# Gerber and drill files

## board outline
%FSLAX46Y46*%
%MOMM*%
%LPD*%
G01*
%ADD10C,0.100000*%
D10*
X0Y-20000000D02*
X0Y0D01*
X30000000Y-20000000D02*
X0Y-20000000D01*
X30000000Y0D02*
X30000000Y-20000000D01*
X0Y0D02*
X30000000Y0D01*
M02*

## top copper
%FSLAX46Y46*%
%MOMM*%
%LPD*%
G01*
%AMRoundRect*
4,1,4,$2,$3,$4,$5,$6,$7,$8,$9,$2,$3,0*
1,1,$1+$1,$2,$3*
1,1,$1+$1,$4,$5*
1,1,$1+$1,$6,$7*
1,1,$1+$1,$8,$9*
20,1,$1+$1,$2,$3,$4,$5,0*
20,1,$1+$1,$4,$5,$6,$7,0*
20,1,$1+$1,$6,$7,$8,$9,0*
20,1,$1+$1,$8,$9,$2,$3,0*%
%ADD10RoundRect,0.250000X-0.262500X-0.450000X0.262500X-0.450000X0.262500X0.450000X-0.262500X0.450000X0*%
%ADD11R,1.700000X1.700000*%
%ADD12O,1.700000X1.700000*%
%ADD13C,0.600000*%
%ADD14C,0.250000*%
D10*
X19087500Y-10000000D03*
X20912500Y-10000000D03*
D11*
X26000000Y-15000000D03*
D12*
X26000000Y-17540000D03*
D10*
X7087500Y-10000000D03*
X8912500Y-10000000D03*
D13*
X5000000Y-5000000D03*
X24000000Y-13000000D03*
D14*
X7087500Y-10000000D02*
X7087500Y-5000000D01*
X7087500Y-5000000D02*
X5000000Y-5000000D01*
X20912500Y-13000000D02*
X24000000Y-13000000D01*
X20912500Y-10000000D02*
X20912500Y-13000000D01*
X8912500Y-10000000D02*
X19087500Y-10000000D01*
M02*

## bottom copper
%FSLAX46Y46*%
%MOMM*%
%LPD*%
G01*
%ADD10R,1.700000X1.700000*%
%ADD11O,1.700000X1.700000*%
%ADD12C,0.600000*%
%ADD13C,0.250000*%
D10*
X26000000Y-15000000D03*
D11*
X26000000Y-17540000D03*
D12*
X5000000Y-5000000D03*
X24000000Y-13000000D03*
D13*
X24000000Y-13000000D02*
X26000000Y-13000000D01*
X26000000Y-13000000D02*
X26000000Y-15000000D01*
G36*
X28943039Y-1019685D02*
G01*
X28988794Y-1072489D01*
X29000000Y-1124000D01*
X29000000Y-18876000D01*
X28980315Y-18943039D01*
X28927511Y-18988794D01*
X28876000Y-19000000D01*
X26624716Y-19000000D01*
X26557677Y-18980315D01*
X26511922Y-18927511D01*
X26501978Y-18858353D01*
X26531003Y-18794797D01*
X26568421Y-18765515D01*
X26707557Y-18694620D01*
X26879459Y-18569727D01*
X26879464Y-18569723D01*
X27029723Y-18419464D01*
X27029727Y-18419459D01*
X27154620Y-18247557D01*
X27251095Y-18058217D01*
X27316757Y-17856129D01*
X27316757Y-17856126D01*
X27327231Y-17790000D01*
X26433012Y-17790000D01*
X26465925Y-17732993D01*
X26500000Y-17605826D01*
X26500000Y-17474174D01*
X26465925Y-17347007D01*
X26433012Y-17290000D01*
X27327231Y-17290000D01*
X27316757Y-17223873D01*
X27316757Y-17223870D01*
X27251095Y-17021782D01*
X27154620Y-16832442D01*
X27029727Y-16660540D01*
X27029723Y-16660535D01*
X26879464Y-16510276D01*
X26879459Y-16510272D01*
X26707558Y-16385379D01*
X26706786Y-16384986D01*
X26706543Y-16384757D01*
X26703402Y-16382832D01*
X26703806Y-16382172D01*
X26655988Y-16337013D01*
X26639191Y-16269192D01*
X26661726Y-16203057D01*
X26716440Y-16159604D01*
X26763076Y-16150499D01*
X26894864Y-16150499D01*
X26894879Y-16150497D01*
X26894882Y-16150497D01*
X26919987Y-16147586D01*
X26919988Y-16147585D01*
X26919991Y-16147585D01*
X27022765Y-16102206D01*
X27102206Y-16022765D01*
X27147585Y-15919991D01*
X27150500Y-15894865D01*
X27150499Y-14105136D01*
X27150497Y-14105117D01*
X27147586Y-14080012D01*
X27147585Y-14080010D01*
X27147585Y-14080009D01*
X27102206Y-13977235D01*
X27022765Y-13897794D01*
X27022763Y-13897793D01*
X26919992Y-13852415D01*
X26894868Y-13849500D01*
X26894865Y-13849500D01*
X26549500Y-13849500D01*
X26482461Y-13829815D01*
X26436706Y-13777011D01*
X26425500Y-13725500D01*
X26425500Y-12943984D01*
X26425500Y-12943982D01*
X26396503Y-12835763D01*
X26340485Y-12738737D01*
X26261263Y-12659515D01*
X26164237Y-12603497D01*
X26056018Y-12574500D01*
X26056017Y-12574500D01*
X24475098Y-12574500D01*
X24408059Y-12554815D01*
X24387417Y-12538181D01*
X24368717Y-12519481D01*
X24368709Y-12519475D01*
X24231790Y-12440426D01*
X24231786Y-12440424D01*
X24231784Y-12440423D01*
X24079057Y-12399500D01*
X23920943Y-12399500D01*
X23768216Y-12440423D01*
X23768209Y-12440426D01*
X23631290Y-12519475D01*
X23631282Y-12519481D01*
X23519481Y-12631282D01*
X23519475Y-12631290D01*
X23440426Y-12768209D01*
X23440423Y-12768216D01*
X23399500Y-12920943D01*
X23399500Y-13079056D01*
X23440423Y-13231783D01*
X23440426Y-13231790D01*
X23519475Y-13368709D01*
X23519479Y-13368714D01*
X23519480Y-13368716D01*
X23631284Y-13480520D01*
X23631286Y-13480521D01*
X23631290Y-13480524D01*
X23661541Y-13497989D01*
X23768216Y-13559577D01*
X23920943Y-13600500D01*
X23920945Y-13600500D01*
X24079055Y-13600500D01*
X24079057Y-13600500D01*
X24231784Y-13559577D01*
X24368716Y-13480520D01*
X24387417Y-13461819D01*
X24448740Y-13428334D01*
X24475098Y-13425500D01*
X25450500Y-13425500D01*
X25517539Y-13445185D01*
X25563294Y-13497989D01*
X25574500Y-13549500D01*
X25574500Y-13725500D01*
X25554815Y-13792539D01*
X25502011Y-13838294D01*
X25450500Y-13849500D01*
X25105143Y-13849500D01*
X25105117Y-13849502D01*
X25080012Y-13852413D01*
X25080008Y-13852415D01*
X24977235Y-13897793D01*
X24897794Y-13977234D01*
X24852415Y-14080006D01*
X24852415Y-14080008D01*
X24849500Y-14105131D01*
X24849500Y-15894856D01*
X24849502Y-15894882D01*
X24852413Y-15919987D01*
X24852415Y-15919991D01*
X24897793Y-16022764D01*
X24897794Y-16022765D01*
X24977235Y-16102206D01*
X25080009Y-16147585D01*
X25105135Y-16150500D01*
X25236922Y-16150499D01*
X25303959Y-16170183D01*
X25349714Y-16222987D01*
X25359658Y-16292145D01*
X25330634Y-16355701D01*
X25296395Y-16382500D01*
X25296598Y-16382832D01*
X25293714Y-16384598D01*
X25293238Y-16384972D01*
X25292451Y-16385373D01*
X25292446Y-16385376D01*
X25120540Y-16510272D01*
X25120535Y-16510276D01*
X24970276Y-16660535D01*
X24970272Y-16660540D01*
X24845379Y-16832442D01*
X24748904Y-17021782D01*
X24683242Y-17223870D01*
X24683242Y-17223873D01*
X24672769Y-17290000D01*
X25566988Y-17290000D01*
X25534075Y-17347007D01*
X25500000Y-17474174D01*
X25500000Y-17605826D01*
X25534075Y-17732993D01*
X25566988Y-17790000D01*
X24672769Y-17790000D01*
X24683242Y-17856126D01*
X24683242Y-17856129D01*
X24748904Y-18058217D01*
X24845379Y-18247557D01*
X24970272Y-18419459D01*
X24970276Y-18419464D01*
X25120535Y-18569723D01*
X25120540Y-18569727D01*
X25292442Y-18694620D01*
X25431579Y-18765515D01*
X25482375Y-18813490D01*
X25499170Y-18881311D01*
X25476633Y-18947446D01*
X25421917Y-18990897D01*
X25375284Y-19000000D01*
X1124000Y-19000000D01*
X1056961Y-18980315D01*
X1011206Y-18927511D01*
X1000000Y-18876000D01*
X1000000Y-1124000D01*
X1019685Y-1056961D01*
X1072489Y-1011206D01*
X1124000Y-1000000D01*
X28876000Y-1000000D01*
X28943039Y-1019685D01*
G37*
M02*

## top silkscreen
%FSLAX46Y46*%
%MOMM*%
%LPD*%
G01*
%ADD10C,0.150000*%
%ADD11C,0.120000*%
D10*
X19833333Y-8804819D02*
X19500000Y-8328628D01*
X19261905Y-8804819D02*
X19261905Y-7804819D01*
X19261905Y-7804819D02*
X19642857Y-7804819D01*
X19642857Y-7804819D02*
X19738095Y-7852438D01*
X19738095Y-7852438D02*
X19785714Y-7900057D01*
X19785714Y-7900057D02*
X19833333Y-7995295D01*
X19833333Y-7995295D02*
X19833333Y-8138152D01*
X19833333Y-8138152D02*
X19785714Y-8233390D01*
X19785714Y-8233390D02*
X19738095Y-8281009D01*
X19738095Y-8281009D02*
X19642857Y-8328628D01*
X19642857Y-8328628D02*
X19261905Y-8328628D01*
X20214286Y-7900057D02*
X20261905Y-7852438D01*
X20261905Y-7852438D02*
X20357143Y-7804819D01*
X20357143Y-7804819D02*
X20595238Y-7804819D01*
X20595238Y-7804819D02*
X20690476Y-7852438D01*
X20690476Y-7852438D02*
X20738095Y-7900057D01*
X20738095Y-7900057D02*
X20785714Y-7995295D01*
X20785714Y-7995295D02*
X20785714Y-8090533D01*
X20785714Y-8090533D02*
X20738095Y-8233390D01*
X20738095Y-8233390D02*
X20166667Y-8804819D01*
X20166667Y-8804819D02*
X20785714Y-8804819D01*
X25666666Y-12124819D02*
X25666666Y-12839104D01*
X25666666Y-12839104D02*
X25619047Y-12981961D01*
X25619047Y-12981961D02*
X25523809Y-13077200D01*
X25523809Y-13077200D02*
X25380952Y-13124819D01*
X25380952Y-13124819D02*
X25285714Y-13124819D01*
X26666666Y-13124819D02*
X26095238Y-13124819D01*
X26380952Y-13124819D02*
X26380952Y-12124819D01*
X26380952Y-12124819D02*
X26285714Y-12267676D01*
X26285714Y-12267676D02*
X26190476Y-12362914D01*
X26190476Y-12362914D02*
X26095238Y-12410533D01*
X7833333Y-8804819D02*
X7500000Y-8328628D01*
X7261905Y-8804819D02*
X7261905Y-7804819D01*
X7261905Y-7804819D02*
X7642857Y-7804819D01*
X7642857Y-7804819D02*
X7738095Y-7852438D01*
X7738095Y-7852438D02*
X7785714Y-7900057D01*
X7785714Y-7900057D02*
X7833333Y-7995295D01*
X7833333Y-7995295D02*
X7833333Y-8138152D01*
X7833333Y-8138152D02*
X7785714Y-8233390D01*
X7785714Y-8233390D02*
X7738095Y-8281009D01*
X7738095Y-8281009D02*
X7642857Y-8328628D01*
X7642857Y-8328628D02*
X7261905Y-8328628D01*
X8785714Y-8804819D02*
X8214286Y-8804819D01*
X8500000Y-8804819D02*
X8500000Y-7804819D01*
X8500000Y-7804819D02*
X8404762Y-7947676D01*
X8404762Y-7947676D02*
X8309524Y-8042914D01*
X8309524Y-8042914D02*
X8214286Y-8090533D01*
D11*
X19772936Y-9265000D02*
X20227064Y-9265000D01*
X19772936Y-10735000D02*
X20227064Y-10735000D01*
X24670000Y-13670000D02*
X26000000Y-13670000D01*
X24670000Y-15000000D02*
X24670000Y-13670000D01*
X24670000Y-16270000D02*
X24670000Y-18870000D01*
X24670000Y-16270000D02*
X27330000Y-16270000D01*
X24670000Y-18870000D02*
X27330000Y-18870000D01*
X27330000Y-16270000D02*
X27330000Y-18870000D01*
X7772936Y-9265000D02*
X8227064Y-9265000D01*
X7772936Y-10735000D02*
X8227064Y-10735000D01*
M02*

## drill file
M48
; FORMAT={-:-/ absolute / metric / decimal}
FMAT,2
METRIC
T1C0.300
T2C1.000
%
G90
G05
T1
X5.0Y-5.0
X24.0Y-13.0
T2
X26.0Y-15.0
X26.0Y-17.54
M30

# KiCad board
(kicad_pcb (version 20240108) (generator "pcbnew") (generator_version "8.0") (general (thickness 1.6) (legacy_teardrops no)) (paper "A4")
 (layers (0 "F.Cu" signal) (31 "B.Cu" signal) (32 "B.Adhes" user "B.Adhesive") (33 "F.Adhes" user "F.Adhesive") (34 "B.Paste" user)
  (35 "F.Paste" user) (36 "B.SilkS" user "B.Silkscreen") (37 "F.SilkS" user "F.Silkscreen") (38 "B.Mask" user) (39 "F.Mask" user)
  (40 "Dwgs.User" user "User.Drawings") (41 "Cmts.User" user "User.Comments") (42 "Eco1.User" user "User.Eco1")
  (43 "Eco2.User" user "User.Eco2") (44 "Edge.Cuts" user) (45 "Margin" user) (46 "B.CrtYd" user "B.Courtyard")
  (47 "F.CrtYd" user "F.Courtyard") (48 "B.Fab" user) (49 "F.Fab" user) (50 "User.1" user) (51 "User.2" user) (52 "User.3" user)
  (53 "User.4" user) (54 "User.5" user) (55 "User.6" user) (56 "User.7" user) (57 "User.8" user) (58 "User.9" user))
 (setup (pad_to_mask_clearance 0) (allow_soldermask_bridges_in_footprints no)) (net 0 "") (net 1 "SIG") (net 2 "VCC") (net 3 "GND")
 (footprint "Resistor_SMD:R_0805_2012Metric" (layer "F.Cu") (at 20 10)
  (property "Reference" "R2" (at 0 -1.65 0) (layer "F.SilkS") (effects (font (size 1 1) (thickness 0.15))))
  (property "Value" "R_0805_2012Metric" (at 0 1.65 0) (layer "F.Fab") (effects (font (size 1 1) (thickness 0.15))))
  (fp_line (start -0.227064 -0.735) (end 0.227064 -0.735) (stroke (width 0.12) (type solid)) (layer "F.SilkS"))
  (fp_line (start -0.227064 0.735) (end 0.227064 0.735) (stroke (width 0.12) (type solid)) (layer "F.SilkS"))
  (pad "1" smd roundrect (at -0.9125 0) (size 1.025 1.4) (layers "F.Cu" "F.Paste" "F.Mask") (roundrect_rratio 0.243902) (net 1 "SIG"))
  (pad "2" smd roundrect (at 0.9125 0) (size 1.025 1.4) (layers "F.Cu" "F.Paste" "F.Mask") (roundrect_rratio 0.243902) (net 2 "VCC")))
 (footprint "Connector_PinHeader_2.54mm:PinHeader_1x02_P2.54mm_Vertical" (layer "F.Cu") (at 26 15)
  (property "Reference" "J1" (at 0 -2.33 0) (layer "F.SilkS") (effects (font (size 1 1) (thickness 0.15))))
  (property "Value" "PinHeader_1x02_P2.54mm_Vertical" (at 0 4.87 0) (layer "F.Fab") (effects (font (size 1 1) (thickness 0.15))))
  (fp_line (start -1.33 -1.33) (end 0 -1.33) (stroke (width 0.12) (type solid)) (layer "F.SilkS"))
  (fp_line (start -1.33 0) (end -1.33 -1.33) (stroke (width 0.12) (type solid)) (layer "F.SilkS"))
  (fp_line (start -1.33 1.27) (end -1.33 3.87) (stroke (width 0.12) (type solid)) (layer "F.SilkS"))
  (fp_line (start -1.33 1.27) (end 1.33 1.27) (stroke (width 0.12) (type solid)) (layer "F.SilkS"))
  (fp_line (start -1.33 3.87) (end 1.33 3.87) (stroke (width 0.12) (type solid)) (layer "F.SilkS"))
  (fp_line (start 1.33 1.27) (end 1.33 3.87) (stroke (width 0.12) (type solid)) (layer "F.SilkS"))
  (pad "1" thru_hole rect (at 0 0) (size 1.7 1.7) (drill 1) (layers "*.Cu" "*.Mask") (remove_unused_layers no) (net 2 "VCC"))
  (pad "2" thru_hole oval (at 0 2.54) (size 1.7 1.7) (drill 1) (layers "*.Cu" "*.Mask") (remove_unused_layers no) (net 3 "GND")))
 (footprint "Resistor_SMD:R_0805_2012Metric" (layer "F.Cu") (at 8 10)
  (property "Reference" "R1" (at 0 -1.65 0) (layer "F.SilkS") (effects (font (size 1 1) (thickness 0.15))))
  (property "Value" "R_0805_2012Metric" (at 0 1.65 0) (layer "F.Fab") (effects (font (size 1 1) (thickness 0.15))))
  (fp_line (start -0.227064 -0.735) (end 0.227064 -0.735) (stroke (width 0.12) (type solid)) (layer "F.SilkS"))
  (fp_line (start -0.227064 0.735) (end 0.227064 0.735) (stroke (width 0.12) (type solid)) (layer "F.SilkS"))
  (pad "1" smd roundrect (at -0.9125 0) (size 1.025 1.4) (layers "F.Cu" "F.Paste" "F.Mask") (roundrect_rratio 0.243902) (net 3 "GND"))
  (pad "2" smd roundrect (at 0.9125 0) (size 1.025 1.4) (layers "F.Cu" "F.Paste" "F.Mask") (roundrect_rratio 0.243902) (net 1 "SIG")))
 (gr_line (start 0 20) (end 0 0) (stroke (width 0.1) (type default)) (layer "Edge.Cuts"))
 (gr_line (start 30 20) (end 0 20) (stroke (width 0.1) (type default)) (layer "Edge.Cuts"))
 (gr_line (start 30 0) (end 30 20) (stroke (width 0.1) (type default)) (layer "Edge.Cuts"))
 (gr_line (start 0 0) (end 30 0) (stroke (width 0.1) (type default)) (layer "Edge.Cuts"))
 (segment (start 7.0875 10) (end 7.0875 5) (width 0.25) (layer "F.Cu") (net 3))
 (segment (start 7.0875 5) (end 5 5) (width 0.25) (layer "F.Cu") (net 3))
 (via (at 5 5) (size 0.6) (drill 0.3) (layers "F.Cu" "B.Cu") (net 3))
 (segment (start 20.9125 13) (end 24 13) (width 0.25) (layer "F.Cu") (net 2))
 (segment (start 20.9125 10) (end 20.9125 13) (width 0.25) (layer "F.Cu") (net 2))
 (via (at 24 13) (size 0.6) (drill 0.3) (layers "F.Cu" "B.Cu") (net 2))
 (segment (start 24 13) (end 26 13) (width 0.25) (layer "B.Cu") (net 2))
 (segment (start 26 13) (end 26 15) (width 0.25) (layer "B.Cu") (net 2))
 (segment (start 8.9125 10) (end 19.0875 10) (width 0.25) (layer "F.Cu") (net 1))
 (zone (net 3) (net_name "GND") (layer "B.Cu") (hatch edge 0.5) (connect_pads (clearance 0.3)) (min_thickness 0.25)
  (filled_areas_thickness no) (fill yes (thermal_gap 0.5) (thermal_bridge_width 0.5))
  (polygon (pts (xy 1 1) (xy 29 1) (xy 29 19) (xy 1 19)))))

